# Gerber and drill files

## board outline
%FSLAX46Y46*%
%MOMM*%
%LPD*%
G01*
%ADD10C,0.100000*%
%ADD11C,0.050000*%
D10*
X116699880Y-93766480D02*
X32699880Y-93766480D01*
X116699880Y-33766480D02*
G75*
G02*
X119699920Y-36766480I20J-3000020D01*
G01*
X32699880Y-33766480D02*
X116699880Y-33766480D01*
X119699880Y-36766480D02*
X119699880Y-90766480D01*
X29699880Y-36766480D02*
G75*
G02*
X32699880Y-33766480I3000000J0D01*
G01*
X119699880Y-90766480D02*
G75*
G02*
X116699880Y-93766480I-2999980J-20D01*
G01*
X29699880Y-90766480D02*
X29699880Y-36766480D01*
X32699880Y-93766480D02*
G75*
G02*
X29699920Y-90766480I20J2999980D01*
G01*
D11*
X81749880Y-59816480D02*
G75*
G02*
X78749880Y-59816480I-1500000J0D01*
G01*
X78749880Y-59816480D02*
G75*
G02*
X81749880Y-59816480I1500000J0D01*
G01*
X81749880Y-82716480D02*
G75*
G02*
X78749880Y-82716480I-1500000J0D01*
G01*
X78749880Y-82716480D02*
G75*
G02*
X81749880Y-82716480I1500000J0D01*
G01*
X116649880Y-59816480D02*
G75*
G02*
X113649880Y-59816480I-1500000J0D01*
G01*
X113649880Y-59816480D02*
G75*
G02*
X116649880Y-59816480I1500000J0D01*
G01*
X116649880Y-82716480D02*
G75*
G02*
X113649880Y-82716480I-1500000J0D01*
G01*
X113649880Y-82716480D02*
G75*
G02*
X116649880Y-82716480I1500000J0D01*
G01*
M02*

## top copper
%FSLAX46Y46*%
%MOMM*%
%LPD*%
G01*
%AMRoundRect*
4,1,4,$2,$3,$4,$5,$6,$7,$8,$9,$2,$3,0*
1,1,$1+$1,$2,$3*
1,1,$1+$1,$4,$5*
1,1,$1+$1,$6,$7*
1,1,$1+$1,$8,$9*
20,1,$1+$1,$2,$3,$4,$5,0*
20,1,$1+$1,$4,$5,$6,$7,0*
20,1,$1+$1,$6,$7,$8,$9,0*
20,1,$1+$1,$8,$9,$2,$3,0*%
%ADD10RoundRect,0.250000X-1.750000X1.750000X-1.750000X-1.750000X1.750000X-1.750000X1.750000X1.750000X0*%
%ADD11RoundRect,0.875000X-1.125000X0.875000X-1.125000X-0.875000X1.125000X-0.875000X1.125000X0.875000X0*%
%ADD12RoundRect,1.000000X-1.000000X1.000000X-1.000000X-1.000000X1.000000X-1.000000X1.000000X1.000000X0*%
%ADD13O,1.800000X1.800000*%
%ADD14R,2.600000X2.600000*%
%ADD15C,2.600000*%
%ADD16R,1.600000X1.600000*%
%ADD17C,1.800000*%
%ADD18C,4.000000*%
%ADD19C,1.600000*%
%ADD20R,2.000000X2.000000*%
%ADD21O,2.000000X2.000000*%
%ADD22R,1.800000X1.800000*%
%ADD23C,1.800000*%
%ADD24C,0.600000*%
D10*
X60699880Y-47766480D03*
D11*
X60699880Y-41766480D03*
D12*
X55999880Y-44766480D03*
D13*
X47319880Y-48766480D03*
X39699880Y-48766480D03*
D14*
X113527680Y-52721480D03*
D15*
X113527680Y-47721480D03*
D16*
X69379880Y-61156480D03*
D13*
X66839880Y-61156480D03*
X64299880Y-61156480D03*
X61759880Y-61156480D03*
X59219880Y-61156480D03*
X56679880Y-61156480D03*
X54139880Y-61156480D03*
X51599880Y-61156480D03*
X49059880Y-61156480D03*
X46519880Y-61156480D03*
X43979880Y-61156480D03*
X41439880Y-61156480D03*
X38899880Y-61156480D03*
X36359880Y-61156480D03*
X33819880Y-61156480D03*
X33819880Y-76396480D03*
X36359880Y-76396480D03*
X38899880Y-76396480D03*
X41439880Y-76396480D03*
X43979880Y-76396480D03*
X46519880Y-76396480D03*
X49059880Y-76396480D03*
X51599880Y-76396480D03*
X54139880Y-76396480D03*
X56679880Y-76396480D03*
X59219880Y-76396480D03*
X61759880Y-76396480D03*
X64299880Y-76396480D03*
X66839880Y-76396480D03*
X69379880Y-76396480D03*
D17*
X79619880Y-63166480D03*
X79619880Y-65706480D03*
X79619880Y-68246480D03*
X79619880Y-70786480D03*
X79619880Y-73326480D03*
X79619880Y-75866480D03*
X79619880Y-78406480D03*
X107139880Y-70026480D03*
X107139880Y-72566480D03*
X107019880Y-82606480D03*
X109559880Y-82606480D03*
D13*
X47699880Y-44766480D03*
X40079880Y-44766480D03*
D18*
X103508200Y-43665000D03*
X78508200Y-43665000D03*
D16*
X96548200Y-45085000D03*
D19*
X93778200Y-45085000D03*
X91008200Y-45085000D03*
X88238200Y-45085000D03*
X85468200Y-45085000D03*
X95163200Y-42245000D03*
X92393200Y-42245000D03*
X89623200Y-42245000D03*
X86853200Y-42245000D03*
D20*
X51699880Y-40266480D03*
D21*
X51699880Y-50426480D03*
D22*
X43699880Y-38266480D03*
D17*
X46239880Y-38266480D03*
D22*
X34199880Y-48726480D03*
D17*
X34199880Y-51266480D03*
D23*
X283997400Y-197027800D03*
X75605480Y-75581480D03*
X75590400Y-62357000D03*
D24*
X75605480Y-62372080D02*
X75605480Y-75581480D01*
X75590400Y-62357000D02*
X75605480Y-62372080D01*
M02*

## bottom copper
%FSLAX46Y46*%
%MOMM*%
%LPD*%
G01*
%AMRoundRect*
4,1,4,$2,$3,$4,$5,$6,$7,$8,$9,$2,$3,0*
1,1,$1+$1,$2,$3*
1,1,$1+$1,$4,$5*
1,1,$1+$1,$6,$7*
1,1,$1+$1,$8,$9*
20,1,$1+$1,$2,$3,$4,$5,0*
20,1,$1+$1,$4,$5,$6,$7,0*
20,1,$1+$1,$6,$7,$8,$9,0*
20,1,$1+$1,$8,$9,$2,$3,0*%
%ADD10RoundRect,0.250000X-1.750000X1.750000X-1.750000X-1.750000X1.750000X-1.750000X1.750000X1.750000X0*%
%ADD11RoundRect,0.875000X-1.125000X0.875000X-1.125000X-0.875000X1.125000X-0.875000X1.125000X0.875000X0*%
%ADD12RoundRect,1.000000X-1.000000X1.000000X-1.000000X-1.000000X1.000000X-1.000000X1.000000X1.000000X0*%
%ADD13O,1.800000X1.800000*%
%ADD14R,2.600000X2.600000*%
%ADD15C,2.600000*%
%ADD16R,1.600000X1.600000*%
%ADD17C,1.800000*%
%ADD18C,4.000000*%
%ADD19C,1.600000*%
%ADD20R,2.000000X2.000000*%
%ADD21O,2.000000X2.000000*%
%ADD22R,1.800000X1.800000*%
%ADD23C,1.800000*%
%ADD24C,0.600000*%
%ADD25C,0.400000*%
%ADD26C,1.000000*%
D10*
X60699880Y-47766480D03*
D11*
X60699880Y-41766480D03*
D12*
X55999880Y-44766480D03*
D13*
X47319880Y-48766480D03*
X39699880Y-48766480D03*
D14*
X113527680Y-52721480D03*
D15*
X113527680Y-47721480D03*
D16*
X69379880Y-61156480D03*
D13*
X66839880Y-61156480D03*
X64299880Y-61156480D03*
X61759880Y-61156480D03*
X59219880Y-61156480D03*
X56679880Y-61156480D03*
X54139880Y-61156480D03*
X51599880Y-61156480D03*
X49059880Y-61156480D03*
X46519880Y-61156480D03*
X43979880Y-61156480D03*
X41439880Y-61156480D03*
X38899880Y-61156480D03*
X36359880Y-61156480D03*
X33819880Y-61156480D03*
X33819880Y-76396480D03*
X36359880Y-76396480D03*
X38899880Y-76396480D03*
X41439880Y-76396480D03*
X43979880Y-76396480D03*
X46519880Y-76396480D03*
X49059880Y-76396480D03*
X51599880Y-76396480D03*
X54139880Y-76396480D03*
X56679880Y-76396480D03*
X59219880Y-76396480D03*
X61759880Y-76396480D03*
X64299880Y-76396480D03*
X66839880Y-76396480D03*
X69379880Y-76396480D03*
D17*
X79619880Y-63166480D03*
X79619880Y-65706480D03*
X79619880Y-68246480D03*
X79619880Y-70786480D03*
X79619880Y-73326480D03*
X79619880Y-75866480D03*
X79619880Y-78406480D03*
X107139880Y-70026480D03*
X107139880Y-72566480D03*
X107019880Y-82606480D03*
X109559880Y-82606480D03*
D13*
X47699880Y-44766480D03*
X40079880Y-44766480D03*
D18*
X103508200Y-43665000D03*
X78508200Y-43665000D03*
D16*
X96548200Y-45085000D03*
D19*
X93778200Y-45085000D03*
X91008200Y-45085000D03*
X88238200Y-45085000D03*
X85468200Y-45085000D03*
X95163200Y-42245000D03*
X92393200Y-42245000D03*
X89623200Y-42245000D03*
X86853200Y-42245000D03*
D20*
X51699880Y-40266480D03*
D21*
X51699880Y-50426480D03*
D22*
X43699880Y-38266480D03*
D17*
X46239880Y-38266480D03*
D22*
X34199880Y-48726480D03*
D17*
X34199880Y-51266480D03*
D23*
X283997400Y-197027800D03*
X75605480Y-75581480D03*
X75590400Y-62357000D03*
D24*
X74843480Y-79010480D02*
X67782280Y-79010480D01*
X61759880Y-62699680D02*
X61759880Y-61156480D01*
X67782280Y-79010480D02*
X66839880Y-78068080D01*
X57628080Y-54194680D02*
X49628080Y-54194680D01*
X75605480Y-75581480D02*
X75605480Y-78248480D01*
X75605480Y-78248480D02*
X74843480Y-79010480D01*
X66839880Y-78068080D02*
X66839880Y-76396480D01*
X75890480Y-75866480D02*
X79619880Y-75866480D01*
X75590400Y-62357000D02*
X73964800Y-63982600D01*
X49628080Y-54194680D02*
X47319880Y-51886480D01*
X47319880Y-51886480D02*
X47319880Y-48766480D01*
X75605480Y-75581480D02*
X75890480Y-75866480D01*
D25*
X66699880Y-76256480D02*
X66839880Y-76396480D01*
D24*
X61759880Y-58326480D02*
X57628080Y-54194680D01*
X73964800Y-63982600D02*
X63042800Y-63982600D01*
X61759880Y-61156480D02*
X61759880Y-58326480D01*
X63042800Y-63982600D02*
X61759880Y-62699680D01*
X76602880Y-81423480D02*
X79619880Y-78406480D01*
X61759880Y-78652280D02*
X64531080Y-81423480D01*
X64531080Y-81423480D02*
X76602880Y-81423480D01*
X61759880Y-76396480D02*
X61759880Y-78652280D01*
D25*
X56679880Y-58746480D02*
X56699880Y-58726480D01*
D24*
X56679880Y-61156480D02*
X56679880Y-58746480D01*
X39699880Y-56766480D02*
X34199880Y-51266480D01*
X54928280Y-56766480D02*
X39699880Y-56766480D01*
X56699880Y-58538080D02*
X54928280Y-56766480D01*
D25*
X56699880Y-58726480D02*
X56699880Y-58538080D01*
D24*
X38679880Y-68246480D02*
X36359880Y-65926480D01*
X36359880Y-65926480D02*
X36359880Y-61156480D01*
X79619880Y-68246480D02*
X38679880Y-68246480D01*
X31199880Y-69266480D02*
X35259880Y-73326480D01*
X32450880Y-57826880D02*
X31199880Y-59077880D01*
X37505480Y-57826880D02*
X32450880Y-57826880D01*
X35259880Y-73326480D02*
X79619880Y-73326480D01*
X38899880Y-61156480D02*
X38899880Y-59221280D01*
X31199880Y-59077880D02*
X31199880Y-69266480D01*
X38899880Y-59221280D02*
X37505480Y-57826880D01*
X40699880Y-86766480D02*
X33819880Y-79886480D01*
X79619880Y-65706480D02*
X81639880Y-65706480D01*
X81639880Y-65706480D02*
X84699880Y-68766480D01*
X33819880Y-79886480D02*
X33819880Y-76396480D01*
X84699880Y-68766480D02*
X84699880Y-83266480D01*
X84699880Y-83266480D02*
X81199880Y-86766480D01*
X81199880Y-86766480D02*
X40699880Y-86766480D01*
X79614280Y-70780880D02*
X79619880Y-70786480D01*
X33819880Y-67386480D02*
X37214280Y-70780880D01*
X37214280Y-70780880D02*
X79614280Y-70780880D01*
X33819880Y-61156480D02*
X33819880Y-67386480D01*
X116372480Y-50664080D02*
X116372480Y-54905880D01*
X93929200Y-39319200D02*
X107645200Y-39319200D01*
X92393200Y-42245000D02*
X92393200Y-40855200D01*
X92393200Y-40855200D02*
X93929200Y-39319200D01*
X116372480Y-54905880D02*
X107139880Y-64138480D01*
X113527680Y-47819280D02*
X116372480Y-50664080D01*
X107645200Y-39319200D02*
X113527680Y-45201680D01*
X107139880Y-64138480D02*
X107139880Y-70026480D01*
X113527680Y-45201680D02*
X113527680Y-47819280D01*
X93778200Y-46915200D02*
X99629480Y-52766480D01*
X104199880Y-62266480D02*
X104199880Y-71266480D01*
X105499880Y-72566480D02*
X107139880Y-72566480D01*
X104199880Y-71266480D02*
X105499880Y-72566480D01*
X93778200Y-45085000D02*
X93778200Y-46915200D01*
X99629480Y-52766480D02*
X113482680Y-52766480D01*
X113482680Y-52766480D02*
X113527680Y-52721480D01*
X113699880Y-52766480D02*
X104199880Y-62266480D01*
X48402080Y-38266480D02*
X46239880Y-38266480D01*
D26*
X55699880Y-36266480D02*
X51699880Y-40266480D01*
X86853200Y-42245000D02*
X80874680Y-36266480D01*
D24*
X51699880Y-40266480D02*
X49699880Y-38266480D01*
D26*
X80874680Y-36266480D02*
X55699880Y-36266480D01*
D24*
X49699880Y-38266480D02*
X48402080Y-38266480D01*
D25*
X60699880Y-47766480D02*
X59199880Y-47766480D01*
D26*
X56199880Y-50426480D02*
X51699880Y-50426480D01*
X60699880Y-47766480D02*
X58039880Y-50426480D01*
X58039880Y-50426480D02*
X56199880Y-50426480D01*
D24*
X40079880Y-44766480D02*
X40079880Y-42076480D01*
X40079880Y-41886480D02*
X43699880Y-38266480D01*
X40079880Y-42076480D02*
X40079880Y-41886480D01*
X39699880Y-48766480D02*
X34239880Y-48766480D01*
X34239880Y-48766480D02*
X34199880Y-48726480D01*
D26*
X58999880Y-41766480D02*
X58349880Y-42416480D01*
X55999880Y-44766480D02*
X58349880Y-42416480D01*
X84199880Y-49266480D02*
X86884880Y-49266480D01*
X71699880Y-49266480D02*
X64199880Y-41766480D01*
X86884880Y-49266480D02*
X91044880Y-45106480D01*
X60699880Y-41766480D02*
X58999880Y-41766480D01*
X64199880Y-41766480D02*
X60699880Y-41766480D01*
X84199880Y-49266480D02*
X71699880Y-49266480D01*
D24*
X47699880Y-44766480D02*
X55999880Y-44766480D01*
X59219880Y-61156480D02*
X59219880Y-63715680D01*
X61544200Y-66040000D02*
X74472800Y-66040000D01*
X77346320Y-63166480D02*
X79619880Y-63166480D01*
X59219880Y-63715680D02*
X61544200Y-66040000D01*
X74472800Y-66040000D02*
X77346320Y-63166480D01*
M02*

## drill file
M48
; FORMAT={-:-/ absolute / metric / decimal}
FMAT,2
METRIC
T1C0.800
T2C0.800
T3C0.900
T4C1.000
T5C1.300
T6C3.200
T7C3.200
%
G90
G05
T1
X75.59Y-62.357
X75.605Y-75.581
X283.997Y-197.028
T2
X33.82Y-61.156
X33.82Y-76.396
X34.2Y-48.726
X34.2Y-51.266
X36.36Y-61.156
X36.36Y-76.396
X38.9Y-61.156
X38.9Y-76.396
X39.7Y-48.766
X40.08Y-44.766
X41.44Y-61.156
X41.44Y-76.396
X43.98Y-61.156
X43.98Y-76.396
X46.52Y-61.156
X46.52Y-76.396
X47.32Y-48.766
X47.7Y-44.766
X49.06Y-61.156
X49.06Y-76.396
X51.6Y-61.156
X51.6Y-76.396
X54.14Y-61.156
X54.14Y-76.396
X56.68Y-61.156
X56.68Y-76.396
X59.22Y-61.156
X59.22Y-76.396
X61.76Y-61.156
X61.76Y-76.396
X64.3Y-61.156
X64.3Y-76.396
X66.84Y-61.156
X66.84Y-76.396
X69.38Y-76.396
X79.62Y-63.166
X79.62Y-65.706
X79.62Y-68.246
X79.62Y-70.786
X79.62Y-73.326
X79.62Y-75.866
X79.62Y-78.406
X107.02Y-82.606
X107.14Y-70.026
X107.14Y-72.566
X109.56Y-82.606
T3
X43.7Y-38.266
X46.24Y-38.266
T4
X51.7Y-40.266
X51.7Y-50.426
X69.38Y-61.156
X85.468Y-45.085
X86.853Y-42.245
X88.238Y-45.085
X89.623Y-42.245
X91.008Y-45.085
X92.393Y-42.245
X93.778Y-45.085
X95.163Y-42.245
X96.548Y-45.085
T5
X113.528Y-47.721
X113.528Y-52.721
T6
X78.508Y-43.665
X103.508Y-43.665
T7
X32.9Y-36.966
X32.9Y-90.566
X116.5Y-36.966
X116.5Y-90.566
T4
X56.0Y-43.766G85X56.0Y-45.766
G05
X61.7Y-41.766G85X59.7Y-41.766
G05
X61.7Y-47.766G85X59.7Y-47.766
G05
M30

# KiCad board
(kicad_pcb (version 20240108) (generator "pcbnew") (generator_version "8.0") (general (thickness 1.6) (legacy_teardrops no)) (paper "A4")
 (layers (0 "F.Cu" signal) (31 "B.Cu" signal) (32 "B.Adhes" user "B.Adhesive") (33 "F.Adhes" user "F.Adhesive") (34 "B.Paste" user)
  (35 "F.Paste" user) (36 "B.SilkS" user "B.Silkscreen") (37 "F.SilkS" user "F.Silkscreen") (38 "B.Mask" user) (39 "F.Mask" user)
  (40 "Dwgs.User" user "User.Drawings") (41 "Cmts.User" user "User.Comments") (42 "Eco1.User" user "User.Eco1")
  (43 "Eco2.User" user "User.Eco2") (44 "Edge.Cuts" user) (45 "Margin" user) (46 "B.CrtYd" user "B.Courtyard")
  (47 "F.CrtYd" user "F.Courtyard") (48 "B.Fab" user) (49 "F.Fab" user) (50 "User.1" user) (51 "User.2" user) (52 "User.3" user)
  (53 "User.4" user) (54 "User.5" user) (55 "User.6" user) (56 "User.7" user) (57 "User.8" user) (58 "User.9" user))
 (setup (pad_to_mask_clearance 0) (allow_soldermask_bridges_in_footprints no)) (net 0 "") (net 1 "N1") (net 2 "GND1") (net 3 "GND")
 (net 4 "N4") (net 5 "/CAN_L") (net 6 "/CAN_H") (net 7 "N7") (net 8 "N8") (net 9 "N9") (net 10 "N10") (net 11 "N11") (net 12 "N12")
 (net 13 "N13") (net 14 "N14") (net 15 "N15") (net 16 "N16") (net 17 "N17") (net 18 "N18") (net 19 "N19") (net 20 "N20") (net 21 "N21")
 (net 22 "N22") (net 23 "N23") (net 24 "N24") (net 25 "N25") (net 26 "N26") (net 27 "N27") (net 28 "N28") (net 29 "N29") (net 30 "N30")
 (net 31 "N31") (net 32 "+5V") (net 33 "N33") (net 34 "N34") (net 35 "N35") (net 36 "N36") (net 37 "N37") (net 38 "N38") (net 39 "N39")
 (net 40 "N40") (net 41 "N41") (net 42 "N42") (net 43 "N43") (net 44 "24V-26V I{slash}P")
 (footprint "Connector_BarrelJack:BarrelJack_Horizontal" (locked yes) (layer "F.Cu") (at 60.69988 47.76648 -90)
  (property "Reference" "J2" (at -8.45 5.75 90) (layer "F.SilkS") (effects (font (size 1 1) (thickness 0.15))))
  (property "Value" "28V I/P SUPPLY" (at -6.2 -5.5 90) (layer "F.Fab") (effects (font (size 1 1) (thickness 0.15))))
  (pad "1" thru_hole roundrect (at 0 0 270) (size 4 4) (drill oval 1 3) (layers "*.Cu" "*.Mask") (remove_unused_layers no)
   (roundrect_rratio 0.0625) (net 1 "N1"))
  (pad "2" thru_hole roundrect (at -6 0 270) (size 3.5 4) (drill oval 1 3) (layers "*.Cu" "*.Mask") (remove_unused_layers no)
   (roundrect_rratio 0.25) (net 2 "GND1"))
  (pad "3" thru_hole roundrect (at -3 4.7 270) (size 4 4) (drill oval 3 1) (layers "*.Cu" "*.Mask") (remove_unused_layers no)
   (roundrect_rratio 0.25) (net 2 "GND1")))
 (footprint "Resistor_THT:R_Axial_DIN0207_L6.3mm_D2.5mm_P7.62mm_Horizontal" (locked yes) (layer "F.Cu") (at 47.31988 48.76648 180)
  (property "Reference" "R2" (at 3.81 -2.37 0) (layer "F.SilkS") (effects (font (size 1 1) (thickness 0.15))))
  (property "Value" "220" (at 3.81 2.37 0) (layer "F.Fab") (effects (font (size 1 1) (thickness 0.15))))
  (pad "1" thru_hole oval (at 0 0 180) (size 1.8 1.8) (drill 0.8) (layers "*.Cu" "*.Mask") (remove_unused_layers no) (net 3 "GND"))
  (pad "2" thru_hole oval (at 7.62 0 180) (size 1.8 1.8) (drill 0.8) (layers "*.Cu" "*.Mask") (remove_unused_layers no) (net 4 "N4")))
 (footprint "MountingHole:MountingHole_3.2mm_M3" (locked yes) (layer "F.Cu") (at 116.49988 36.96648)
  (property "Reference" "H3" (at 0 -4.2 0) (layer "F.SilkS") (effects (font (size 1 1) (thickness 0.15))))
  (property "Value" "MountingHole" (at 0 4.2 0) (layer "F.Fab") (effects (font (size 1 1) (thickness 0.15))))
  (pad "" np_thru_hole circle (at 0 0) (size 3.2 3.2) (drill 3.2) (layers "*.Cu" "*.Mask")))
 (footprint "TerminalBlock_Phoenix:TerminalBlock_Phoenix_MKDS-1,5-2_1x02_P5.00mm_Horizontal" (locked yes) (layer "F.Cu")
  (at 113.52768 52.72148 90)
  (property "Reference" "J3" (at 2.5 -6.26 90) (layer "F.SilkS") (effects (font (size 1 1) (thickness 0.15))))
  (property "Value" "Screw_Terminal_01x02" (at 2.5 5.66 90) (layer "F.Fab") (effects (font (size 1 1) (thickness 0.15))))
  (pad "1" thru_hole rect (at 0 0 90) (size 2.6 2.6) (drill 1.3) (layers "*.Cu" "*.Mask") (remove_unused_layers no) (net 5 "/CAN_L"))
  (pad "2" thru_hole circle (at 5 0 90) (size 2.6 2.6) (drill 1.3) (layers "*.Cu" "*.Mask") (remove_unused_layers no) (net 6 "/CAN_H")))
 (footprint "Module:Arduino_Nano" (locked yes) (layer "F.Cu") (at 69.37988 61.15648 -90)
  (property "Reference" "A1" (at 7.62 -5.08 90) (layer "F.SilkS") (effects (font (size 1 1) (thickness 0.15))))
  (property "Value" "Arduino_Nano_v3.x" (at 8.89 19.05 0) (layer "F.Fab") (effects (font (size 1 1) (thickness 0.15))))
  (pad "1" thru_hole rect (at 0 0 270) (size 1.6 1.6) (drill 1) (layers "*.Cu" "*.Mask") (remove_unused_layers no) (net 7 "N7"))
  (pad "2" thru_hole oval (at 0 2.54 270) (size 1.8 1.8) (drill 0.8) (layers "*.Cu" "*.Mask") (remove_unused_layers no) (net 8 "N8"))
  (pad "3" thru_hole oval (at 0 5.08 270) (size 1.8 1.8) (drill 0.8) (layers "*.Cu" "*.Mask") (remove_unused_layers no) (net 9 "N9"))
  (pad "4" thru_hole oval (at 0 7.62 270) (size 1.8 1.8) (drill 0.8) (layers "*.Cu" "*.Mask") (remove_unused_layers no) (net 3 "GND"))
  (pad "5" thru_hole oval (at 0 10.16 270) (size 1.8 1.8) (drill 0.8) (layers "*.Cu" "*.Mask") (remove_unused_layers no) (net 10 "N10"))
  (pad "6" thru_hole oval (at 0 12.7 270) (size 1.8 1.8) (drill 0.8) (layers "*.Cu" "*.Mask") (remove_unused_layers no) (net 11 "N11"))
  (pad "7" thru_hole oval (at 0 15.24 270) (size 1.8 1.8) (drill 0.8) (layers "*.Cu" "*.Mask") (remove_unused_layers no) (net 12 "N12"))
  (pad "8" thru_hole oval (at 0 17.78 270) (size 1.8 1.8) (drill 0.8) (layers "*.Cu" "*.Mask") (remove_unused_layers no) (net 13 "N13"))
  (pad "9" thru_hole oval (at 0 20.32 270) (size 1.8 1.8) (drill 0.8) (layers "*.Cu" "*.Mask") (remove_unused_layers no) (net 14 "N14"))
  (pad "10" thru_hole oval (at 0 22.86 270) (size 1.8 1.8) (drill 0.8) (layers "*.Cu" "*.Mask") (remove_unused_layers no) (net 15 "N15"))
  (pad "11" thru_hole oval (at 0 25.4 270) (size 1.8 1.8) (drill 0.8) (layers "*.Cu" "*.Mask") (remove_unused_layers no) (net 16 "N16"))
  (pad "12" thru_hole oval (at 0 27.94 270) (size 1.8 1.8) (drill 0.8) (layers "*.Cu" "*.Mask") (remove_unused_layers no) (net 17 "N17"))
  (pad "13" thru_hole oval (at 0 30.48 270) (size 1.8 1.8) (drill 0.8) (layers "*.Cu" "*.Mask") (remove_unused_layers no) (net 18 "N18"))
  (pad "14" thru_hole oval (at 0 33.02 270) (size 1.8 1.8) (drill 0.8) (layers "*.Cu" "*.Mask") (remove_unused_layers no) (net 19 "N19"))
  (pad "15" thru_hole oval (at 0 35.56 270) (size 1.8 1.8) (drill 0.8) (layers "*.Cu" "*.Mask") (remove_unused_layers no) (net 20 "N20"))
  (pad "16" thru_hole oval (at 15.24 35.56 270) (size 1.8 1.8) (drill 0.8) (layers "*.Cu" "*.Mask") (remove_unused_layers no) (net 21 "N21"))
  (pad "17" thru_hole oval (at 15.24 33.02 270) (size 1.8 1.8) (drill 0.8) (layers "*.Cu" "*.Mask") (remove_unused_layers no) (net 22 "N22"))
  (pad "18" thru_hole oval (at 15.24 30.48 270) (size 1.8 1.8) (drill 0.8) (layers "*.Cu" "*.Mask") (remove_unused_layers no) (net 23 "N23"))
  (pad "19" thru_hole oval (at 15.24 27.94 270) (size 1.8 1.8) (drill 0.8) (layers "*.Cu" "*.Mask") (remove_unused_layers no) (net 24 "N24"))
  (pad "20" thru_hole oval (at 15.24 25.4 270) (size 1.8 1.8) (drill 0.8) (layers "*.Cu" "*.Mask") (remove_unused_layers no) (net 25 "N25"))
  (pad "21" thru_hole oval (at 15.24 22.86 270) (size 1.8 1.8) (drill 0.8) (layers "*.Cu" "*.Mask") (remove_unused_layers no) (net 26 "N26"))
  (pad "22" thru_hole oval (at 15.24 20.32 270) (size 1.8 1.8) (drill 0.8) (layers "*.Cu" "*.Mask") (remove_unused_layers no) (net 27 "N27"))
  (pad "23" thru_hole oval (at 15.24 17.78 270) (size 1.8 1.8) (drill 0.8) (layers "*.Cu" "*.Mask") (remove_unused_layers no) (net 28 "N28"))
  (pad "24" thru_hole oval (at 15.24 15.24 270) (size 1.8 1.8) (drill 0.8) (layers "*.Cu" "*.Mask") (remove_unused_layers no) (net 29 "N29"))
  (pad "25" thru_hole oval (at 15.24 12.7 270) (size 1.8 1.8) (drill 0.8) (layers "*.Cu" "*.Mask") (remove_unused_layers no) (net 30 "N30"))
  (pad "26" thru_hole oval (at 15.24 10.16 270) (size 1.8 1.8) (drill 0.8) (layers "*.Cu" "*.Mask") (remove_unused_layers no) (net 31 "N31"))
  (pad "27" thru_hole oval (at 15.24 7.62 270) (size 1.8 1.8) (drill 0.8) (layers "*.Cu" "*.Mask") (remove_unused_layers no) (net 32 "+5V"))
  (pad "28" thru_hole oval (at 15.24 5.08 270) (size 1.8 1.8) (drill 0.8) (layers "*.Cu" "*.Mask") (remove_unused_layers no) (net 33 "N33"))
  (pad "29" thru_hole oval (at 15.24 2.54 270) (size 1.8 1.8) (drill 0.8) (layers "*.Cu" "*.Mask") (remove_unused_layers no) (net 3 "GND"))
  (pad "30" thru_hole oval (at 15.24 0 270) (size 1.8 1.8) (drill 0.8) (layers "*.Cu" "*.Mask") (remove_unused_layers no) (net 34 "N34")))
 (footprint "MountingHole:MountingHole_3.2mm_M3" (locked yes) (layer "F.Cu") (at 32.89988 90.56648)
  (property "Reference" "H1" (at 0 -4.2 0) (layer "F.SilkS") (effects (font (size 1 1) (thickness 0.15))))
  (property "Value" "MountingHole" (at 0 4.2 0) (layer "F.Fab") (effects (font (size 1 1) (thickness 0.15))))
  (pad "" np_thru_hole circle (at 0 0) (size 3.2 3.2) (drill 3.2) (layers "*.Cu" "*.Mask")))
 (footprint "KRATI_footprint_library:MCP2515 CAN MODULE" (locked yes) (layer "F.Cu") (at 97.39988 69.64648)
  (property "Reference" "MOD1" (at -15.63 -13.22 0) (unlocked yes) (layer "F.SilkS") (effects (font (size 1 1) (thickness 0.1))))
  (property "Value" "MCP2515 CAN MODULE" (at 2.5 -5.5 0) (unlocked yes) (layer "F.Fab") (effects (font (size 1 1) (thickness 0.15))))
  (fp_circle (center -17.15 -9.83) (end -15.65 -9.83) (stroke (width 0.05) (type default)) (fill none) (layer "Edge.Cuts"))
  (fp_circle (center -17.15 13.07) (end -15.65 13.07) (stroke (width 0.05) (type default)) (fill none) (layer "Edge.Cuts"))
  (fp_circle (center 17.75 -9.83) (end 19.25 -9.83) (stroke (width 0.05) (type default)) (fill none) (layer "Edge.Cuts"))
  (fp_circle (center 17.75 13.07) (end 19.25 13.07) (stroke (width 0.05) (type default)) (fill none) (layer "Edge.Cuts"))
  (pad "1" thru_hole circle (at -17.78 -6.48 90) (size 1.8 1.8) (drill 0.8) (layers "*.Cu" "*.Mask") (remove_unused_layers no)
   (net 10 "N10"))
  (pad "2" thru_hole circle (at -17.78 -3.94 90) (size 1.8 1.8) (drill 0.8) (layers "*.Cu" "*.Mask") (remove_unused_layers no)
   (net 21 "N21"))
  (pad "3" thru_hole circle (at -17.78 -1.4 90) (size 1.8 1.8) (drill 0.8) (layers "*.Cu" "*.Mask") (remove_unused_layers no) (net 19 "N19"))
  (pad "4" thru_hole circle (at -17.78 1.14 90) (size 1.8 1.8) (drill 0.8) (layers "*.Cu" "*.Mask") (remove_unused_layers no) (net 20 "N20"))
  (pad "5" thru_hole circle (at -17.78 3.68 90) (size 1.8 1.8) (drill 0.8) (layers "*.Cu" "*.Mask") (remove_unused_layers no) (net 18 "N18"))
  (pad "6" thru_hole circle (at -17.78 6.22 90) (size 1.8 1.8) (drill 0.8) (layers "*.Cu" "*.Mask") (remove_unused_layers no) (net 3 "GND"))
  (pad "7" thru_hole circle (at -17.78 8.76 90) (size 1.8 1.8) (drill 0.8) (layers "*.Cu" "*.Mask") (remove_unused_layers no) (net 32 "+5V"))
  (pad "8" thru_hole circle (at 9.74 0.38 90) (size 1.8 1.8) (drill 0.8) (layers "*.Cu" "*.Mask") (remove_unused_layers no) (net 6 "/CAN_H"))
  (pad "9" thru_hole circle (at 9.74 2.92 90) (size 1.8 1.8) (drill 0.8) (layers "*.Cu" "*.Mask") (remove_unused_layers no) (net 5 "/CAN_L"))
  (pad "10" thru_hole circle (at 9.62 12.96 90) (size 1.8 1.8) (drill 0.8) (layers "*.Cu" "*.Mask") (remove_unused_layers no) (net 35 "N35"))
  (pad "11" thru_hole circle (at 12.16 12.96 90) (size 1.8 1.8) (drill 0.8) (layers "*.Cu" "*.Mask") (remove_unused_layers no)
   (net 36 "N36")))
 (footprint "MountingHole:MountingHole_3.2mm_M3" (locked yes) (layer "F.Cu") (at 32.89988 36.96648)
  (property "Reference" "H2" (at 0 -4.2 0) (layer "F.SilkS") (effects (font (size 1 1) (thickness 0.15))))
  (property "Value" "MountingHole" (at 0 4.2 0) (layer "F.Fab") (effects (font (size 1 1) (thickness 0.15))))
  (pad "" np_thru_hole circle (at 0 0) (size 3.2 3.2) (drill 3.2) (layers "*.Cu" "*.Mask")))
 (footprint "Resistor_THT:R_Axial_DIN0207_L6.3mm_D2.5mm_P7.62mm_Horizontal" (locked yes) (layer "F.Cu") (at 47.69988 44.76648 180)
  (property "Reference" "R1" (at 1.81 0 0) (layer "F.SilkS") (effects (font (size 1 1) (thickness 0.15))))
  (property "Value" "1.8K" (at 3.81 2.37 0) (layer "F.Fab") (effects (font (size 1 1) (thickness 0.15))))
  (pad "1" thru_hole oval (at 0 0 180) (size 1.8 1.8) (drill 0.8) (layers "*.Cu" "*.Mask") (remove_unused_layers no) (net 2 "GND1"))
  (pad "2" thru_hole oval (at 7.62 0 180) (size 1.8 1.8) (drill 0.8) (layers "*.Cu" "*.Mask") (remove_unused_layers no) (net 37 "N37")))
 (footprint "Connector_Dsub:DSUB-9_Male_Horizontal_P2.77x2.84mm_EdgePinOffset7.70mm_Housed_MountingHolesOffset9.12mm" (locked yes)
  (layer "F.Cu") (at 96.5482 45.085 180)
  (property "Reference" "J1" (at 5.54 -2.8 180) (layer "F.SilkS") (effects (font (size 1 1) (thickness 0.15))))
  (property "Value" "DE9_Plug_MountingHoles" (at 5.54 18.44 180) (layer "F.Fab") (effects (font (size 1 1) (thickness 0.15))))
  (pad "0" thru_hole circle (at -6.96 1.42 180) (size 4 4) (drill 3.2) (layers "*.Cu" "*.Mask") (remove_unused_layers no) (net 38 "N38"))
  (pad "0" thru_hole circle (at 18.04 1.42 180) (size 4 4) (drill 3.2) (layers "*.Cu" "*.Mask") (remove_unused_layers no) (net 38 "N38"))
  (pad "1" thru_hole rect (at 0 0 180) (size 1.6 1.6) (drill 1) (layers "*.Cu" "*.Mask") (remove_unused_layers no) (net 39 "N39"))
  (pad "2" thru_hole circle (at 2.77 0 180) (size 1.6 1.6) (drill 1) (layers "*.Cu" "*.Mask") (remove_unused_layers no) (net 5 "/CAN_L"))
  (pad "3" thru_hole circle (at 5.54 0 180) (size 1.6 1.6) (drill 1) (layers "*.Cu" "*.Mask") (remove_unused_layers no) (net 2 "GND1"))
  (pad "4" thru_hole circle (at 8.31 0 180) (size 1.6 1.6) (drill 1) (layers "*.Cu" "*.Mask") (remove_unused_layers no) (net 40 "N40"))
  (pad "5" thru_hole circle (at 11.08 0 180) (size 1.6 1.6) (drill 1) (layers "*.Cu" "*.Mask") (remove_unused_layers no) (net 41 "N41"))
  (pad "6" thru_hole circle (at 1.385 2.84 180) (size 1.6 1.6) (drill 1) (layers "*.Cu" "*.Mask") (remove_unused_layers no) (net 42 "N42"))
  (pad "7" thru_hole circle (at 4.155 2.84 180) (size 1.6 1.6) (drill 1) (layers "*.Cu" "*.Mask") (remove_unused_layers no) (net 6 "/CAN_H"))
  (pad "8" thru_hole circle (at 6.925 2.84 180) (size 1.6 1.6) (drill 1) (layers "*.Cu" "*.Mask") (remove_unused_layers no) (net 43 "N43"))
  (pad "9" thru_hole circle (at 9.695 2.84 180) (size 1.6 1.6) (drill 1) (layers "*.Cu" "*.Mask") (remove_unused_layers no)
   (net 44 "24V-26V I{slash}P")))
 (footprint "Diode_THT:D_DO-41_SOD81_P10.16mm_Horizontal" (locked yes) (layer "F.Cu") (at 51.69988 40.26648 -90)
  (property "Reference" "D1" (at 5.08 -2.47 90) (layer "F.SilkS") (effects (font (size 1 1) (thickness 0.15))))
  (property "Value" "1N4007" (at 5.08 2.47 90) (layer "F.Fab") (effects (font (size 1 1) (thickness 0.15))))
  (pad "1" thru_hole rect (at 0 0 270) (size 2 2) (drill 1) (layers "*.Cu" "*.Mask") (remove_unused_layers no) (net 44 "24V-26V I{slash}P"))
  (pad "2" thru_hole oval (at 10.16 0 270) (size 2 2) (drill 1) (layers "*.Cu" "*.Mask") (remove_unused_layers no) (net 1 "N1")))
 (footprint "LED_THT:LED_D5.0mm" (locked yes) (layer "F.Cu") (at 43.69988 38.26648)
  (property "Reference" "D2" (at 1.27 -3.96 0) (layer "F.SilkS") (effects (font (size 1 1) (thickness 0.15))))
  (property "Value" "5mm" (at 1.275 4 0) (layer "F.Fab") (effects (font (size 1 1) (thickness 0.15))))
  (pad "1" thru_hole rect (at 0 0) (size 1.8 1.8) (drill 0.9) (layers "*.Cu" "*.Mask") (remove_unused_layers no) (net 37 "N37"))
  (pad "2" thru_hole circle (at 2.54 0) (size 1.8 1.8) (drill 0.9) (layers "*.Cu" "*.Mask") (remove_unused_layers no)
   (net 44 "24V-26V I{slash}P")))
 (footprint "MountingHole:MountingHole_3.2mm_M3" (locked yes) (layer "F.Cu") (at 116.49988 90.56648)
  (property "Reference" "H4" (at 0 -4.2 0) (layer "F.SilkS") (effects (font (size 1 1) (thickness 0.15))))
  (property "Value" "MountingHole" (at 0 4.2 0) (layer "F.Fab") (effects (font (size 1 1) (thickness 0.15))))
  (pad "" np_thru_hole circle (at 0 0) (size 3.2 3.2) (drill 3.2) (layers "*.Cu" "*.Mask")))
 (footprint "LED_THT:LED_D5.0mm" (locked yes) (layer "F.Cu") (at 34.19988 48.72648 -90)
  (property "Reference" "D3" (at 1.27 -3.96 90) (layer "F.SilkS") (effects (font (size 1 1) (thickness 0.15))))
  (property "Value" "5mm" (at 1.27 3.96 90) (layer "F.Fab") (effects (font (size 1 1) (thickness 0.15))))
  (pad "1" thru_hole rect (at 0 0 270) (size 1.8 1.8) (drill 0.8) (layers "*.Cu" "*.Mask") (remove_unused_layers no) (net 4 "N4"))
  (pad "2" thru_hole circle (at 2.54 0 270) (size 1.8 1.8) (drill 0.8) (layers "*.Cu" "*.Mask") (remove_unused_layers no) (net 11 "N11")))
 (gr_line (start 116.69988 93.76648) (end 32.69988 93.76648) (locked yes) (stroke (width 0.1) (type default)) (layer "Edge.Cuts"))
 (gr_arc (start 116.69988 33.76648) (mid 118.8212 34.64516) (end 119.69988 36.76648) (locked yes) (stroke (width 0.1) (type default))
  (layer "Edge.Cuts"))
 (gr_line (start 32.69988 33.76648) (end 116.69988 33.76648) (locked yes) (stroke (width 0.1) (type default)) (layer "Edge.Cuts"))
 (gr_line (start 119.69988 36.76648) (end 119.69988 90.76648) (locked yes) (stroke (width 0.1) (type default)) (layer "Edge.Cuts"))
 (gr_arc (start 29.69988 36.76648) (mid 30.57856 34.64516) (end 32.69988 33.76648) (locked yes) (stroke (width 0.1) (type default))
  (layer "Edge.Cuts"))
 (gr_arc (start 119.69988 90.76648) (mid 118.8212 92.8878) (end 116.69988 93.76648) (locked yes) (stroke (width 0.1) (type default))
  (layer "Edge.Cuts"))
 (gr_line (start 29.69988 90.76648) (end 29.69988 36.76648) (locked yes) (stroke (width 0.1) (type default)) (layer "Edge.Cuts"))
 (gr_arc (start 32.69988 93.76648) (mid 30.57856 92.8878) (end 29.69988 90.76648) (locked yes) (stroke (width 0.1) (type default))
  (layer "Edge.Cuts"))
 (via (at 283.9974 197.0278) (size 1.8) (drill 0.8) (layers "F.Cu" "B.Cu") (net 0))
 (segment (start 75.60548 62.37208) (end 75.60548 75.58148) (width 0.6) (locked yes) (layer "F.Cu") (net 3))
 (segment (start 75.5904 62.357) (end 75.60548 62.37208) (width 0.6) (locked yes) (layer "F.Cu") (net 3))
 (via (at 75.60548 75.58148) (size 1.8) (drill 0.8) (layers "F.Cu" "B.Cu") (locked yes) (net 3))
 (via (at 75.5904 62.357) (size 1.8) (drill 0.8) (layers "F.Cu" "B.Cu") (locked yes) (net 3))
 (segment (start 74.84348 79.01048) (end 67.78228 79.01048) (width 0.6) (locked yes) (layer "B.Cu") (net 3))
 (segment (start 61.75988 62.69968) (end 61.75988 61.15648) (width 0.6) (locked yes) (layer "B.Cu") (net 3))
 (segment (start 67.78228 79.01048) (end 66.83988 78.06808) (width 0.6) (locked yes) (layer "B.Cu") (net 3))
 (segment (start 57.62808 54.19468) (end 49.62808 54.19468) (width 0.6) (locked yes) (layer "B.Cu") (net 3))
 (segment (start 75.60548 75.58148) (end 75.60548 78.24848) (width 0.6) (locked yes) (layer "B.Cu") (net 3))
 (segment (start 75.60548 78.24848) (end 74.84348 79.01048) (width 0.6) (locked yes) (layer "B.Cu") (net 3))
 (segment (start 66.83988 78.06808) (end 66.83988 76.39648) (width 0.6) (locked yes) (layer "B.Cu") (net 3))
 (segment (start 75.89048 75.86648) (end 79.61988 75.86648) (width 0.6) (locked yes) (layer "B.Cu") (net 3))
 (segment (start 75.5904 62.357) (end 73.9648 63.9826) (width 0.6) (locked yes) (layer "B.Cu") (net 3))
 (segment (start 49.62808 54.19468) (end 47.31988 51.88648) (width 0.6) (locked yes) (layer "B.Cu") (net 3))
 (segment (start 47.31988 51.88648) (end 47.31988 48.76648) (width 0.6) (locked yes) (layer "B.Cu") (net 3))
 (segment (start 75.60548 75.58148) (end 75.89048 75.86648) (width 0.6) (locked yes) (layer "B.Cu") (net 3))
 (segment (start 66.69988 76.25648) (end 66.83988 76.39648) (width 0.4) (locked yes) (layer "B.Cu") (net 3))
 (segment (start 61.75988 58.32648) (end 57.62808 54.19468) (width 0.6) (locked yes) (layer "B.Cu") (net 3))
 (segment (start 73.9648 63.9826) (end 63.0428 63.9826) (width 0.6) (locked yes) (layer "B.Cu") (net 3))
 (segment (start 61.75988 61.15648) (end 61.75988 58.32648) (width 0.6) (locked yes) (layer "B.Cu") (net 3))
 (segment (start 63.0428 63.9826) (end 61.75988 62.69968) (width 0.6) (locked yes) (layer "B.Cu") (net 3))
 (segment (start 76.60288 81.42348) (end 79.61988 78.40648) (width 0.6) (locked yes) (layer "B.Cu") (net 32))
 (segment (start 61.75988 78.65228) (end 64.53108 81.42348) (width 0.6) (locked yes) (layer "B.Cu") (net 32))
 (segment (start 64.53108 81.42348) (end 76.60288 81.42348) (width 0.6) (locked yes) (layer "B.Cu") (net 32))
 (segment (start 61.75988 76.39648) (end 61.75988 78.65228) (width 0.6) (locked yes) (layer "B.Cu") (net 32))
 (segment (start 56.67988 58.74648) (end 56.69988 58.72648) (width 0.4) (locked yes) (layer "B.Cu") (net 11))
 (segment (start 56.67988 61.15648) (end 56.67988 58.74648) (width 0.6) (locked yes) (layer "B.Cu") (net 11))
 (segment (start 39.69988 56.76648) (end 34.19988 51.26648) (width 0.6) (locked yes) (layer "B.Cu") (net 11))
 (segment (start 54.92828 56.76648) (end 39.69988 56.76648) (width 0.6) (locked yes) (layer "B.Cu") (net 11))
 (segment (start 56.69988 58.53808) (end 54.92828 56.76648) (width 0.6) (locked yes) (layer "B.Cu") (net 11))
 (segment (start 56.69988 58.72648) (end 56.69988 58.53808) (width 0.4) (locked yes) (layer "B.Cu") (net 11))
 (segment (start 38.67988 68.24648) (end 36.35988 65.92648) (width 0.6) (locked yes) (layer "B.Cu") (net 19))
 (segment (start 36.35988 65.92648) (end 36.35988 61.15648) (width 0.6) (locked yes) (layer "B.Cu") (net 19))
 (segment (start 79.61988 68.24648) (end 38.67988 68.24648) (width 0.6) (locked yes) (layer "B.Cu") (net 19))
 (segment (start 31.19988 69.26648) (end 35.25988 73.32648) (width 0.6) (locked yes) (layer "B.Cu") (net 18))
 (segment (start 32.45088 57.82688) (end 31.19988 59.07788) (width 0.6) (locked yes) (layer "B.Cu") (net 18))
 (segment (start 37.50548 57.82688) (end 32.45088 57.82688) (width 0.6) (locked yes) (layer "B.Cu") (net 18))
 (segment (start 35.25988 73.32648) (end 79.61988 73.32648) (width 0.6) (locked yes) (layer "B.Cu") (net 18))
 (segment (start 38.89988 61.15648) (end 38.89988 59.22128) (width 0.6) (locked yes) (layer "B.Cu") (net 18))
 (segment (start 31.19988 59.07788) (end 31.19988 69.26648) (width 0.6) (locked yes) (layer "B.Cu") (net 18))
 (segment (start 38.89988 59.22128) (end 37.50548 57.82688) (width 0.6) (locked yes) (layer "B.Cu") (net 18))
 (segment (start 40.69988 86.76648) (end 33.81988 79.88648) (width 0.6) (locked yes) (layer "B.Cu") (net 21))
 (segment (start 79.61988 65.70648) (end 81.63988 65.70648) (width 0.6) (locked yes) (layer "B.Cu") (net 21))
 (segment (start 81.63988 65.70648) (end 84.69988 68.76648) (width 0.6) (locked yes) (layer "B.Cu") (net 21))
 (segment (start 33.81988 79.88648) (end 33.81988 76.39648) (width 0.6) (locked yes) (layer "B.Cu") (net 21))
 (segment (start 84.69988 68.76648) (end 84.69988 83.26648) (width 0.6) (locked yes) (layer "B.Cu") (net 21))
 (segment (start 84.69988 83.26648) (end 81.19988 86.76648) (width 0.6) (locked yes) (layer "B.Cu") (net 21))
 (segment (start 81.19988 86.76648) (end 40.69988 86.76648) (width 0.6) (locked yes) (layer "B.Cu") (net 21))
 (segment (start 79.61428 70.78088) (end 79.61988 70.78648) (width 0.6) (locked yes) (layer "B.Cu") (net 20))
 (segment (start 33.81988 67.38648) (end 37.21428 70.78088) (width 0.6) (locked yes) (layer "B.Cu") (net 20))
 (segment (start 37.21428 70.78088) (end 79.61428 70.78088) (width 0.6) (locked yes) (layer "B.Cu") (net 20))
 (segment (start 33.81988 61.15648) (end 33.81988 67.38648) (width 0.6) (locked yes) (layer "B.Cu") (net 20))
 (segment (start 116.37248 50.66408) (end 116.37248 54.90588) (width 0.6) (locked yes) (layer "B.Cu") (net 6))
 (segment (start 93.9292 39.3192) (end 107.6452 39.3192) (width 0.6) (locked yes) (layer "B.Cu") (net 6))
 (segment (start 92.3932 42.245) (end 92.3932 40.8552) (width 0.6) (locked yes) (layer "B.Cu") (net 6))
 (segment (start 92.3932 40.8552) (end 93.9292 39.3192) (width 0.6) (locked yes) (layer "B.Cu") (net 6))
 (segment (start 116.37248 54.90588) (end 107.13988 64.13848) (width 0.6) (locked yes) (layer "B.Cu") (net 6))
 (segment (start 113.52768 47.81928) (end 116.37248 50.66408) (width 0.6) (locked yes) (layer "B.Cu") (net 6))
 (segment (start 107.6452 39.3192) (end 113.52768 45.20168) (width 0.6) (locked yes) (layer "B.Cu") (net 6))
 (segment (start 107.13988 64.13848) (end 107.13988 70.02648) (width 0.6) (locked yes) (layer "B.Cu") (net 6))
 (segment (start 113.52768 45.20168) (end 113.52768 47.81928) (width 0.6) (locked yes) (layer "B.Cu") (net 6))
 (segment (start 93.7782 46.9152) (end 99.62948 52.76648) (width 0.6) (locked yes) (layer "B.Cu") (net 5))
 (segment (start 104.19988 62.26648) (end 104.19988 71.26648) (width 0.6) (locked yes) (layer "B.Cu") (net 5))
 (segment (start 105.49988 72.56648) (end 107.13988 72.56648) (width 0.6) (locked yes) (layer "B.Cu") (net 5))
 (segment (start 104.19988 71.26648) (end 105.49988 72.56648) (width 0.6) (locked yes) (layer "B.Cu") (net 5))
 (segment (start 93.7782 45.085) (end 93.7782 46.9152) (width 0.6) (locked yes) (layer "B.Cu") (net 5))
 (segment (start 99.62948 52.76648) (end 113.48268 52.76648) (width 0.6) (locked yes) (layer "B.Cu") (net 5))
 (segment (start 113.48268 52.76648) (end 113.52768 52.72148) (width 0.6) (locked yes) (layer "B.Cu") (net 5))
 (segment (start 113.69988 52.76648) (end 104.19988 62.26648) (width 0.6) (locked yes) (layer "B.Cu") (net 5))
 (segment (start 48.40208 38.26648) (end 46.23988 38.26648) (width 0.6) (locked yes) (layer "B.Cu") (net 44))
 (segment (start 55.69988 36.26648) (end 51.69988 40.26648) (width 1) (locked yes) (layer "B.Cu") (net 44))
 (segment (start 86.8532 42.245) (end 80.87468 36.26648) (width 1) (locked yes) (layer "B.Cu") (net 44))
 (segment (start 51.69988 40.26648) (end 49.69988 38.26648) (width 0.6) (locked yes) (layer "B.Cu") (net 44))
 (segment (start 80.87468 36.26648) (end 55.69988 36.26648) (width 1) (locked yes) (layer "B.Cu") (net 44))
 (segment (start 49.69988 38.26648) (end 48.40208 38.26648) (width 0.6) (locked yes) (layer "B.Cu") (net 44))
 (segment (start 60.69988 47.76648) (end 59.19988 47.76648) (width 0.4) (locked yes) (layer "B.Cu") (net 1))
 (segment (start 56.19988 50.42648) (end 51.69988 50.42648) (width 1) (locked yes) (layer "B.Cu") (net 1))
 (segment (start 60.69988 47.76648) (end 58.03988 50.42648) (width 1) (locked yes) (layer "B.Cu") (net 1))
 (segment (start 58.03988 50.42648) (end 56.19988 50.42648) (width 1) (locked yes) (layer "B.Cu") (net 1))
 (segment (start 40.07988 44.76648) (end 40.07988 42.07648) (width 0.6) (locked yes) (layer "B.Cu") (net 37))
 (segment (start 40.07988 41.88648) (end 43.69988 38.26648) (width 0.6) (locked yes) (layer "B.Cu") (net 37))
 (segment (start 40.07988 42.07648) (end 40.07988 41.88648) (width 0.6) (locked yes) (layer "B.Cu") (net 37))
 (segment (start 39.69988 48.76648) (end 34.23988 48.76648) (width 0.6) (locked yes) (layer "B.Cu") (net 4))
 (segment (start 34.23988 48.76648) (end 34.19988 48.72648) (width 0.6) (locked yes) (layer "B.Cu") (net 4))
 (segment (start 58.99988 41.76648) (end 58.34988 42.41648) (width 1) (locked yes) (layer "B.Cu") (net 2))
 (segment (start 55.99988 44.76648) (end 58.34988 42.41648) (width 1) (locked yes) (layer "B.Cu") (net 2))
 (segment (start 84.19988 49.26648) (end 86.88488 49.26648) (width 1) (locked yes) (layer "B.Cu") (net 2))
 (segment (start 71.69988 49.26648) (end 64.19988 41.76648) (width 1) (locked yes) (layer "B.Cu") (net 2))
 (segment (start 86.88488 49.26648) (end 91.04488 45.10648) (width 1) (locked yes) (layer "B.Cu") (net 2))
 (segment (start 60.69988 41.76648) (end 58.99988 41.76648) (width 1) (locked yes) (layer "B.Cu") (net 2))
 (segment (start 64.19988 41.76648) (end 60.69988 41.76648) (width 1) (locked yes) (layer "B.Cu") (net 2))
 (segment (start 84.19988 49.26648) (end 71.69988 49.26648) (width 1) (locked yes) (layer "B.Cu") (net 2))
 (segment (start 47.69988 44.76648) (end 55.99988 44.76648) (width 0.6) (locked yes) (layer "B.Cu") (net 2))
 (segment (start 59.21988 61.15648) (end 59.21988 63.71568) (width 0.6) (locked yes) (layer "B.Cu") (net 10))
 (segment (start 61.5442 66.04) (end 74.4728 66.04) (width 0.6) (locked yes) (layer "B.Cu") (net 10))
 (segment (start 77.34632 63.16648) (end 79.61988 63.16648) (width 0.6) (locked yes) (layer "B.Cu") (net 10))
 (segment (start 59.21988 63.71568) (end 61.5442 66.04) (width 0.6) (locked yes) (layer "B.Cu") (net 10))
 (segment (start 74.4728 66.04) (end 77.34632 63.16648) (width 0.6) (locked yes) (layer "B.Cu") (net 10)))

